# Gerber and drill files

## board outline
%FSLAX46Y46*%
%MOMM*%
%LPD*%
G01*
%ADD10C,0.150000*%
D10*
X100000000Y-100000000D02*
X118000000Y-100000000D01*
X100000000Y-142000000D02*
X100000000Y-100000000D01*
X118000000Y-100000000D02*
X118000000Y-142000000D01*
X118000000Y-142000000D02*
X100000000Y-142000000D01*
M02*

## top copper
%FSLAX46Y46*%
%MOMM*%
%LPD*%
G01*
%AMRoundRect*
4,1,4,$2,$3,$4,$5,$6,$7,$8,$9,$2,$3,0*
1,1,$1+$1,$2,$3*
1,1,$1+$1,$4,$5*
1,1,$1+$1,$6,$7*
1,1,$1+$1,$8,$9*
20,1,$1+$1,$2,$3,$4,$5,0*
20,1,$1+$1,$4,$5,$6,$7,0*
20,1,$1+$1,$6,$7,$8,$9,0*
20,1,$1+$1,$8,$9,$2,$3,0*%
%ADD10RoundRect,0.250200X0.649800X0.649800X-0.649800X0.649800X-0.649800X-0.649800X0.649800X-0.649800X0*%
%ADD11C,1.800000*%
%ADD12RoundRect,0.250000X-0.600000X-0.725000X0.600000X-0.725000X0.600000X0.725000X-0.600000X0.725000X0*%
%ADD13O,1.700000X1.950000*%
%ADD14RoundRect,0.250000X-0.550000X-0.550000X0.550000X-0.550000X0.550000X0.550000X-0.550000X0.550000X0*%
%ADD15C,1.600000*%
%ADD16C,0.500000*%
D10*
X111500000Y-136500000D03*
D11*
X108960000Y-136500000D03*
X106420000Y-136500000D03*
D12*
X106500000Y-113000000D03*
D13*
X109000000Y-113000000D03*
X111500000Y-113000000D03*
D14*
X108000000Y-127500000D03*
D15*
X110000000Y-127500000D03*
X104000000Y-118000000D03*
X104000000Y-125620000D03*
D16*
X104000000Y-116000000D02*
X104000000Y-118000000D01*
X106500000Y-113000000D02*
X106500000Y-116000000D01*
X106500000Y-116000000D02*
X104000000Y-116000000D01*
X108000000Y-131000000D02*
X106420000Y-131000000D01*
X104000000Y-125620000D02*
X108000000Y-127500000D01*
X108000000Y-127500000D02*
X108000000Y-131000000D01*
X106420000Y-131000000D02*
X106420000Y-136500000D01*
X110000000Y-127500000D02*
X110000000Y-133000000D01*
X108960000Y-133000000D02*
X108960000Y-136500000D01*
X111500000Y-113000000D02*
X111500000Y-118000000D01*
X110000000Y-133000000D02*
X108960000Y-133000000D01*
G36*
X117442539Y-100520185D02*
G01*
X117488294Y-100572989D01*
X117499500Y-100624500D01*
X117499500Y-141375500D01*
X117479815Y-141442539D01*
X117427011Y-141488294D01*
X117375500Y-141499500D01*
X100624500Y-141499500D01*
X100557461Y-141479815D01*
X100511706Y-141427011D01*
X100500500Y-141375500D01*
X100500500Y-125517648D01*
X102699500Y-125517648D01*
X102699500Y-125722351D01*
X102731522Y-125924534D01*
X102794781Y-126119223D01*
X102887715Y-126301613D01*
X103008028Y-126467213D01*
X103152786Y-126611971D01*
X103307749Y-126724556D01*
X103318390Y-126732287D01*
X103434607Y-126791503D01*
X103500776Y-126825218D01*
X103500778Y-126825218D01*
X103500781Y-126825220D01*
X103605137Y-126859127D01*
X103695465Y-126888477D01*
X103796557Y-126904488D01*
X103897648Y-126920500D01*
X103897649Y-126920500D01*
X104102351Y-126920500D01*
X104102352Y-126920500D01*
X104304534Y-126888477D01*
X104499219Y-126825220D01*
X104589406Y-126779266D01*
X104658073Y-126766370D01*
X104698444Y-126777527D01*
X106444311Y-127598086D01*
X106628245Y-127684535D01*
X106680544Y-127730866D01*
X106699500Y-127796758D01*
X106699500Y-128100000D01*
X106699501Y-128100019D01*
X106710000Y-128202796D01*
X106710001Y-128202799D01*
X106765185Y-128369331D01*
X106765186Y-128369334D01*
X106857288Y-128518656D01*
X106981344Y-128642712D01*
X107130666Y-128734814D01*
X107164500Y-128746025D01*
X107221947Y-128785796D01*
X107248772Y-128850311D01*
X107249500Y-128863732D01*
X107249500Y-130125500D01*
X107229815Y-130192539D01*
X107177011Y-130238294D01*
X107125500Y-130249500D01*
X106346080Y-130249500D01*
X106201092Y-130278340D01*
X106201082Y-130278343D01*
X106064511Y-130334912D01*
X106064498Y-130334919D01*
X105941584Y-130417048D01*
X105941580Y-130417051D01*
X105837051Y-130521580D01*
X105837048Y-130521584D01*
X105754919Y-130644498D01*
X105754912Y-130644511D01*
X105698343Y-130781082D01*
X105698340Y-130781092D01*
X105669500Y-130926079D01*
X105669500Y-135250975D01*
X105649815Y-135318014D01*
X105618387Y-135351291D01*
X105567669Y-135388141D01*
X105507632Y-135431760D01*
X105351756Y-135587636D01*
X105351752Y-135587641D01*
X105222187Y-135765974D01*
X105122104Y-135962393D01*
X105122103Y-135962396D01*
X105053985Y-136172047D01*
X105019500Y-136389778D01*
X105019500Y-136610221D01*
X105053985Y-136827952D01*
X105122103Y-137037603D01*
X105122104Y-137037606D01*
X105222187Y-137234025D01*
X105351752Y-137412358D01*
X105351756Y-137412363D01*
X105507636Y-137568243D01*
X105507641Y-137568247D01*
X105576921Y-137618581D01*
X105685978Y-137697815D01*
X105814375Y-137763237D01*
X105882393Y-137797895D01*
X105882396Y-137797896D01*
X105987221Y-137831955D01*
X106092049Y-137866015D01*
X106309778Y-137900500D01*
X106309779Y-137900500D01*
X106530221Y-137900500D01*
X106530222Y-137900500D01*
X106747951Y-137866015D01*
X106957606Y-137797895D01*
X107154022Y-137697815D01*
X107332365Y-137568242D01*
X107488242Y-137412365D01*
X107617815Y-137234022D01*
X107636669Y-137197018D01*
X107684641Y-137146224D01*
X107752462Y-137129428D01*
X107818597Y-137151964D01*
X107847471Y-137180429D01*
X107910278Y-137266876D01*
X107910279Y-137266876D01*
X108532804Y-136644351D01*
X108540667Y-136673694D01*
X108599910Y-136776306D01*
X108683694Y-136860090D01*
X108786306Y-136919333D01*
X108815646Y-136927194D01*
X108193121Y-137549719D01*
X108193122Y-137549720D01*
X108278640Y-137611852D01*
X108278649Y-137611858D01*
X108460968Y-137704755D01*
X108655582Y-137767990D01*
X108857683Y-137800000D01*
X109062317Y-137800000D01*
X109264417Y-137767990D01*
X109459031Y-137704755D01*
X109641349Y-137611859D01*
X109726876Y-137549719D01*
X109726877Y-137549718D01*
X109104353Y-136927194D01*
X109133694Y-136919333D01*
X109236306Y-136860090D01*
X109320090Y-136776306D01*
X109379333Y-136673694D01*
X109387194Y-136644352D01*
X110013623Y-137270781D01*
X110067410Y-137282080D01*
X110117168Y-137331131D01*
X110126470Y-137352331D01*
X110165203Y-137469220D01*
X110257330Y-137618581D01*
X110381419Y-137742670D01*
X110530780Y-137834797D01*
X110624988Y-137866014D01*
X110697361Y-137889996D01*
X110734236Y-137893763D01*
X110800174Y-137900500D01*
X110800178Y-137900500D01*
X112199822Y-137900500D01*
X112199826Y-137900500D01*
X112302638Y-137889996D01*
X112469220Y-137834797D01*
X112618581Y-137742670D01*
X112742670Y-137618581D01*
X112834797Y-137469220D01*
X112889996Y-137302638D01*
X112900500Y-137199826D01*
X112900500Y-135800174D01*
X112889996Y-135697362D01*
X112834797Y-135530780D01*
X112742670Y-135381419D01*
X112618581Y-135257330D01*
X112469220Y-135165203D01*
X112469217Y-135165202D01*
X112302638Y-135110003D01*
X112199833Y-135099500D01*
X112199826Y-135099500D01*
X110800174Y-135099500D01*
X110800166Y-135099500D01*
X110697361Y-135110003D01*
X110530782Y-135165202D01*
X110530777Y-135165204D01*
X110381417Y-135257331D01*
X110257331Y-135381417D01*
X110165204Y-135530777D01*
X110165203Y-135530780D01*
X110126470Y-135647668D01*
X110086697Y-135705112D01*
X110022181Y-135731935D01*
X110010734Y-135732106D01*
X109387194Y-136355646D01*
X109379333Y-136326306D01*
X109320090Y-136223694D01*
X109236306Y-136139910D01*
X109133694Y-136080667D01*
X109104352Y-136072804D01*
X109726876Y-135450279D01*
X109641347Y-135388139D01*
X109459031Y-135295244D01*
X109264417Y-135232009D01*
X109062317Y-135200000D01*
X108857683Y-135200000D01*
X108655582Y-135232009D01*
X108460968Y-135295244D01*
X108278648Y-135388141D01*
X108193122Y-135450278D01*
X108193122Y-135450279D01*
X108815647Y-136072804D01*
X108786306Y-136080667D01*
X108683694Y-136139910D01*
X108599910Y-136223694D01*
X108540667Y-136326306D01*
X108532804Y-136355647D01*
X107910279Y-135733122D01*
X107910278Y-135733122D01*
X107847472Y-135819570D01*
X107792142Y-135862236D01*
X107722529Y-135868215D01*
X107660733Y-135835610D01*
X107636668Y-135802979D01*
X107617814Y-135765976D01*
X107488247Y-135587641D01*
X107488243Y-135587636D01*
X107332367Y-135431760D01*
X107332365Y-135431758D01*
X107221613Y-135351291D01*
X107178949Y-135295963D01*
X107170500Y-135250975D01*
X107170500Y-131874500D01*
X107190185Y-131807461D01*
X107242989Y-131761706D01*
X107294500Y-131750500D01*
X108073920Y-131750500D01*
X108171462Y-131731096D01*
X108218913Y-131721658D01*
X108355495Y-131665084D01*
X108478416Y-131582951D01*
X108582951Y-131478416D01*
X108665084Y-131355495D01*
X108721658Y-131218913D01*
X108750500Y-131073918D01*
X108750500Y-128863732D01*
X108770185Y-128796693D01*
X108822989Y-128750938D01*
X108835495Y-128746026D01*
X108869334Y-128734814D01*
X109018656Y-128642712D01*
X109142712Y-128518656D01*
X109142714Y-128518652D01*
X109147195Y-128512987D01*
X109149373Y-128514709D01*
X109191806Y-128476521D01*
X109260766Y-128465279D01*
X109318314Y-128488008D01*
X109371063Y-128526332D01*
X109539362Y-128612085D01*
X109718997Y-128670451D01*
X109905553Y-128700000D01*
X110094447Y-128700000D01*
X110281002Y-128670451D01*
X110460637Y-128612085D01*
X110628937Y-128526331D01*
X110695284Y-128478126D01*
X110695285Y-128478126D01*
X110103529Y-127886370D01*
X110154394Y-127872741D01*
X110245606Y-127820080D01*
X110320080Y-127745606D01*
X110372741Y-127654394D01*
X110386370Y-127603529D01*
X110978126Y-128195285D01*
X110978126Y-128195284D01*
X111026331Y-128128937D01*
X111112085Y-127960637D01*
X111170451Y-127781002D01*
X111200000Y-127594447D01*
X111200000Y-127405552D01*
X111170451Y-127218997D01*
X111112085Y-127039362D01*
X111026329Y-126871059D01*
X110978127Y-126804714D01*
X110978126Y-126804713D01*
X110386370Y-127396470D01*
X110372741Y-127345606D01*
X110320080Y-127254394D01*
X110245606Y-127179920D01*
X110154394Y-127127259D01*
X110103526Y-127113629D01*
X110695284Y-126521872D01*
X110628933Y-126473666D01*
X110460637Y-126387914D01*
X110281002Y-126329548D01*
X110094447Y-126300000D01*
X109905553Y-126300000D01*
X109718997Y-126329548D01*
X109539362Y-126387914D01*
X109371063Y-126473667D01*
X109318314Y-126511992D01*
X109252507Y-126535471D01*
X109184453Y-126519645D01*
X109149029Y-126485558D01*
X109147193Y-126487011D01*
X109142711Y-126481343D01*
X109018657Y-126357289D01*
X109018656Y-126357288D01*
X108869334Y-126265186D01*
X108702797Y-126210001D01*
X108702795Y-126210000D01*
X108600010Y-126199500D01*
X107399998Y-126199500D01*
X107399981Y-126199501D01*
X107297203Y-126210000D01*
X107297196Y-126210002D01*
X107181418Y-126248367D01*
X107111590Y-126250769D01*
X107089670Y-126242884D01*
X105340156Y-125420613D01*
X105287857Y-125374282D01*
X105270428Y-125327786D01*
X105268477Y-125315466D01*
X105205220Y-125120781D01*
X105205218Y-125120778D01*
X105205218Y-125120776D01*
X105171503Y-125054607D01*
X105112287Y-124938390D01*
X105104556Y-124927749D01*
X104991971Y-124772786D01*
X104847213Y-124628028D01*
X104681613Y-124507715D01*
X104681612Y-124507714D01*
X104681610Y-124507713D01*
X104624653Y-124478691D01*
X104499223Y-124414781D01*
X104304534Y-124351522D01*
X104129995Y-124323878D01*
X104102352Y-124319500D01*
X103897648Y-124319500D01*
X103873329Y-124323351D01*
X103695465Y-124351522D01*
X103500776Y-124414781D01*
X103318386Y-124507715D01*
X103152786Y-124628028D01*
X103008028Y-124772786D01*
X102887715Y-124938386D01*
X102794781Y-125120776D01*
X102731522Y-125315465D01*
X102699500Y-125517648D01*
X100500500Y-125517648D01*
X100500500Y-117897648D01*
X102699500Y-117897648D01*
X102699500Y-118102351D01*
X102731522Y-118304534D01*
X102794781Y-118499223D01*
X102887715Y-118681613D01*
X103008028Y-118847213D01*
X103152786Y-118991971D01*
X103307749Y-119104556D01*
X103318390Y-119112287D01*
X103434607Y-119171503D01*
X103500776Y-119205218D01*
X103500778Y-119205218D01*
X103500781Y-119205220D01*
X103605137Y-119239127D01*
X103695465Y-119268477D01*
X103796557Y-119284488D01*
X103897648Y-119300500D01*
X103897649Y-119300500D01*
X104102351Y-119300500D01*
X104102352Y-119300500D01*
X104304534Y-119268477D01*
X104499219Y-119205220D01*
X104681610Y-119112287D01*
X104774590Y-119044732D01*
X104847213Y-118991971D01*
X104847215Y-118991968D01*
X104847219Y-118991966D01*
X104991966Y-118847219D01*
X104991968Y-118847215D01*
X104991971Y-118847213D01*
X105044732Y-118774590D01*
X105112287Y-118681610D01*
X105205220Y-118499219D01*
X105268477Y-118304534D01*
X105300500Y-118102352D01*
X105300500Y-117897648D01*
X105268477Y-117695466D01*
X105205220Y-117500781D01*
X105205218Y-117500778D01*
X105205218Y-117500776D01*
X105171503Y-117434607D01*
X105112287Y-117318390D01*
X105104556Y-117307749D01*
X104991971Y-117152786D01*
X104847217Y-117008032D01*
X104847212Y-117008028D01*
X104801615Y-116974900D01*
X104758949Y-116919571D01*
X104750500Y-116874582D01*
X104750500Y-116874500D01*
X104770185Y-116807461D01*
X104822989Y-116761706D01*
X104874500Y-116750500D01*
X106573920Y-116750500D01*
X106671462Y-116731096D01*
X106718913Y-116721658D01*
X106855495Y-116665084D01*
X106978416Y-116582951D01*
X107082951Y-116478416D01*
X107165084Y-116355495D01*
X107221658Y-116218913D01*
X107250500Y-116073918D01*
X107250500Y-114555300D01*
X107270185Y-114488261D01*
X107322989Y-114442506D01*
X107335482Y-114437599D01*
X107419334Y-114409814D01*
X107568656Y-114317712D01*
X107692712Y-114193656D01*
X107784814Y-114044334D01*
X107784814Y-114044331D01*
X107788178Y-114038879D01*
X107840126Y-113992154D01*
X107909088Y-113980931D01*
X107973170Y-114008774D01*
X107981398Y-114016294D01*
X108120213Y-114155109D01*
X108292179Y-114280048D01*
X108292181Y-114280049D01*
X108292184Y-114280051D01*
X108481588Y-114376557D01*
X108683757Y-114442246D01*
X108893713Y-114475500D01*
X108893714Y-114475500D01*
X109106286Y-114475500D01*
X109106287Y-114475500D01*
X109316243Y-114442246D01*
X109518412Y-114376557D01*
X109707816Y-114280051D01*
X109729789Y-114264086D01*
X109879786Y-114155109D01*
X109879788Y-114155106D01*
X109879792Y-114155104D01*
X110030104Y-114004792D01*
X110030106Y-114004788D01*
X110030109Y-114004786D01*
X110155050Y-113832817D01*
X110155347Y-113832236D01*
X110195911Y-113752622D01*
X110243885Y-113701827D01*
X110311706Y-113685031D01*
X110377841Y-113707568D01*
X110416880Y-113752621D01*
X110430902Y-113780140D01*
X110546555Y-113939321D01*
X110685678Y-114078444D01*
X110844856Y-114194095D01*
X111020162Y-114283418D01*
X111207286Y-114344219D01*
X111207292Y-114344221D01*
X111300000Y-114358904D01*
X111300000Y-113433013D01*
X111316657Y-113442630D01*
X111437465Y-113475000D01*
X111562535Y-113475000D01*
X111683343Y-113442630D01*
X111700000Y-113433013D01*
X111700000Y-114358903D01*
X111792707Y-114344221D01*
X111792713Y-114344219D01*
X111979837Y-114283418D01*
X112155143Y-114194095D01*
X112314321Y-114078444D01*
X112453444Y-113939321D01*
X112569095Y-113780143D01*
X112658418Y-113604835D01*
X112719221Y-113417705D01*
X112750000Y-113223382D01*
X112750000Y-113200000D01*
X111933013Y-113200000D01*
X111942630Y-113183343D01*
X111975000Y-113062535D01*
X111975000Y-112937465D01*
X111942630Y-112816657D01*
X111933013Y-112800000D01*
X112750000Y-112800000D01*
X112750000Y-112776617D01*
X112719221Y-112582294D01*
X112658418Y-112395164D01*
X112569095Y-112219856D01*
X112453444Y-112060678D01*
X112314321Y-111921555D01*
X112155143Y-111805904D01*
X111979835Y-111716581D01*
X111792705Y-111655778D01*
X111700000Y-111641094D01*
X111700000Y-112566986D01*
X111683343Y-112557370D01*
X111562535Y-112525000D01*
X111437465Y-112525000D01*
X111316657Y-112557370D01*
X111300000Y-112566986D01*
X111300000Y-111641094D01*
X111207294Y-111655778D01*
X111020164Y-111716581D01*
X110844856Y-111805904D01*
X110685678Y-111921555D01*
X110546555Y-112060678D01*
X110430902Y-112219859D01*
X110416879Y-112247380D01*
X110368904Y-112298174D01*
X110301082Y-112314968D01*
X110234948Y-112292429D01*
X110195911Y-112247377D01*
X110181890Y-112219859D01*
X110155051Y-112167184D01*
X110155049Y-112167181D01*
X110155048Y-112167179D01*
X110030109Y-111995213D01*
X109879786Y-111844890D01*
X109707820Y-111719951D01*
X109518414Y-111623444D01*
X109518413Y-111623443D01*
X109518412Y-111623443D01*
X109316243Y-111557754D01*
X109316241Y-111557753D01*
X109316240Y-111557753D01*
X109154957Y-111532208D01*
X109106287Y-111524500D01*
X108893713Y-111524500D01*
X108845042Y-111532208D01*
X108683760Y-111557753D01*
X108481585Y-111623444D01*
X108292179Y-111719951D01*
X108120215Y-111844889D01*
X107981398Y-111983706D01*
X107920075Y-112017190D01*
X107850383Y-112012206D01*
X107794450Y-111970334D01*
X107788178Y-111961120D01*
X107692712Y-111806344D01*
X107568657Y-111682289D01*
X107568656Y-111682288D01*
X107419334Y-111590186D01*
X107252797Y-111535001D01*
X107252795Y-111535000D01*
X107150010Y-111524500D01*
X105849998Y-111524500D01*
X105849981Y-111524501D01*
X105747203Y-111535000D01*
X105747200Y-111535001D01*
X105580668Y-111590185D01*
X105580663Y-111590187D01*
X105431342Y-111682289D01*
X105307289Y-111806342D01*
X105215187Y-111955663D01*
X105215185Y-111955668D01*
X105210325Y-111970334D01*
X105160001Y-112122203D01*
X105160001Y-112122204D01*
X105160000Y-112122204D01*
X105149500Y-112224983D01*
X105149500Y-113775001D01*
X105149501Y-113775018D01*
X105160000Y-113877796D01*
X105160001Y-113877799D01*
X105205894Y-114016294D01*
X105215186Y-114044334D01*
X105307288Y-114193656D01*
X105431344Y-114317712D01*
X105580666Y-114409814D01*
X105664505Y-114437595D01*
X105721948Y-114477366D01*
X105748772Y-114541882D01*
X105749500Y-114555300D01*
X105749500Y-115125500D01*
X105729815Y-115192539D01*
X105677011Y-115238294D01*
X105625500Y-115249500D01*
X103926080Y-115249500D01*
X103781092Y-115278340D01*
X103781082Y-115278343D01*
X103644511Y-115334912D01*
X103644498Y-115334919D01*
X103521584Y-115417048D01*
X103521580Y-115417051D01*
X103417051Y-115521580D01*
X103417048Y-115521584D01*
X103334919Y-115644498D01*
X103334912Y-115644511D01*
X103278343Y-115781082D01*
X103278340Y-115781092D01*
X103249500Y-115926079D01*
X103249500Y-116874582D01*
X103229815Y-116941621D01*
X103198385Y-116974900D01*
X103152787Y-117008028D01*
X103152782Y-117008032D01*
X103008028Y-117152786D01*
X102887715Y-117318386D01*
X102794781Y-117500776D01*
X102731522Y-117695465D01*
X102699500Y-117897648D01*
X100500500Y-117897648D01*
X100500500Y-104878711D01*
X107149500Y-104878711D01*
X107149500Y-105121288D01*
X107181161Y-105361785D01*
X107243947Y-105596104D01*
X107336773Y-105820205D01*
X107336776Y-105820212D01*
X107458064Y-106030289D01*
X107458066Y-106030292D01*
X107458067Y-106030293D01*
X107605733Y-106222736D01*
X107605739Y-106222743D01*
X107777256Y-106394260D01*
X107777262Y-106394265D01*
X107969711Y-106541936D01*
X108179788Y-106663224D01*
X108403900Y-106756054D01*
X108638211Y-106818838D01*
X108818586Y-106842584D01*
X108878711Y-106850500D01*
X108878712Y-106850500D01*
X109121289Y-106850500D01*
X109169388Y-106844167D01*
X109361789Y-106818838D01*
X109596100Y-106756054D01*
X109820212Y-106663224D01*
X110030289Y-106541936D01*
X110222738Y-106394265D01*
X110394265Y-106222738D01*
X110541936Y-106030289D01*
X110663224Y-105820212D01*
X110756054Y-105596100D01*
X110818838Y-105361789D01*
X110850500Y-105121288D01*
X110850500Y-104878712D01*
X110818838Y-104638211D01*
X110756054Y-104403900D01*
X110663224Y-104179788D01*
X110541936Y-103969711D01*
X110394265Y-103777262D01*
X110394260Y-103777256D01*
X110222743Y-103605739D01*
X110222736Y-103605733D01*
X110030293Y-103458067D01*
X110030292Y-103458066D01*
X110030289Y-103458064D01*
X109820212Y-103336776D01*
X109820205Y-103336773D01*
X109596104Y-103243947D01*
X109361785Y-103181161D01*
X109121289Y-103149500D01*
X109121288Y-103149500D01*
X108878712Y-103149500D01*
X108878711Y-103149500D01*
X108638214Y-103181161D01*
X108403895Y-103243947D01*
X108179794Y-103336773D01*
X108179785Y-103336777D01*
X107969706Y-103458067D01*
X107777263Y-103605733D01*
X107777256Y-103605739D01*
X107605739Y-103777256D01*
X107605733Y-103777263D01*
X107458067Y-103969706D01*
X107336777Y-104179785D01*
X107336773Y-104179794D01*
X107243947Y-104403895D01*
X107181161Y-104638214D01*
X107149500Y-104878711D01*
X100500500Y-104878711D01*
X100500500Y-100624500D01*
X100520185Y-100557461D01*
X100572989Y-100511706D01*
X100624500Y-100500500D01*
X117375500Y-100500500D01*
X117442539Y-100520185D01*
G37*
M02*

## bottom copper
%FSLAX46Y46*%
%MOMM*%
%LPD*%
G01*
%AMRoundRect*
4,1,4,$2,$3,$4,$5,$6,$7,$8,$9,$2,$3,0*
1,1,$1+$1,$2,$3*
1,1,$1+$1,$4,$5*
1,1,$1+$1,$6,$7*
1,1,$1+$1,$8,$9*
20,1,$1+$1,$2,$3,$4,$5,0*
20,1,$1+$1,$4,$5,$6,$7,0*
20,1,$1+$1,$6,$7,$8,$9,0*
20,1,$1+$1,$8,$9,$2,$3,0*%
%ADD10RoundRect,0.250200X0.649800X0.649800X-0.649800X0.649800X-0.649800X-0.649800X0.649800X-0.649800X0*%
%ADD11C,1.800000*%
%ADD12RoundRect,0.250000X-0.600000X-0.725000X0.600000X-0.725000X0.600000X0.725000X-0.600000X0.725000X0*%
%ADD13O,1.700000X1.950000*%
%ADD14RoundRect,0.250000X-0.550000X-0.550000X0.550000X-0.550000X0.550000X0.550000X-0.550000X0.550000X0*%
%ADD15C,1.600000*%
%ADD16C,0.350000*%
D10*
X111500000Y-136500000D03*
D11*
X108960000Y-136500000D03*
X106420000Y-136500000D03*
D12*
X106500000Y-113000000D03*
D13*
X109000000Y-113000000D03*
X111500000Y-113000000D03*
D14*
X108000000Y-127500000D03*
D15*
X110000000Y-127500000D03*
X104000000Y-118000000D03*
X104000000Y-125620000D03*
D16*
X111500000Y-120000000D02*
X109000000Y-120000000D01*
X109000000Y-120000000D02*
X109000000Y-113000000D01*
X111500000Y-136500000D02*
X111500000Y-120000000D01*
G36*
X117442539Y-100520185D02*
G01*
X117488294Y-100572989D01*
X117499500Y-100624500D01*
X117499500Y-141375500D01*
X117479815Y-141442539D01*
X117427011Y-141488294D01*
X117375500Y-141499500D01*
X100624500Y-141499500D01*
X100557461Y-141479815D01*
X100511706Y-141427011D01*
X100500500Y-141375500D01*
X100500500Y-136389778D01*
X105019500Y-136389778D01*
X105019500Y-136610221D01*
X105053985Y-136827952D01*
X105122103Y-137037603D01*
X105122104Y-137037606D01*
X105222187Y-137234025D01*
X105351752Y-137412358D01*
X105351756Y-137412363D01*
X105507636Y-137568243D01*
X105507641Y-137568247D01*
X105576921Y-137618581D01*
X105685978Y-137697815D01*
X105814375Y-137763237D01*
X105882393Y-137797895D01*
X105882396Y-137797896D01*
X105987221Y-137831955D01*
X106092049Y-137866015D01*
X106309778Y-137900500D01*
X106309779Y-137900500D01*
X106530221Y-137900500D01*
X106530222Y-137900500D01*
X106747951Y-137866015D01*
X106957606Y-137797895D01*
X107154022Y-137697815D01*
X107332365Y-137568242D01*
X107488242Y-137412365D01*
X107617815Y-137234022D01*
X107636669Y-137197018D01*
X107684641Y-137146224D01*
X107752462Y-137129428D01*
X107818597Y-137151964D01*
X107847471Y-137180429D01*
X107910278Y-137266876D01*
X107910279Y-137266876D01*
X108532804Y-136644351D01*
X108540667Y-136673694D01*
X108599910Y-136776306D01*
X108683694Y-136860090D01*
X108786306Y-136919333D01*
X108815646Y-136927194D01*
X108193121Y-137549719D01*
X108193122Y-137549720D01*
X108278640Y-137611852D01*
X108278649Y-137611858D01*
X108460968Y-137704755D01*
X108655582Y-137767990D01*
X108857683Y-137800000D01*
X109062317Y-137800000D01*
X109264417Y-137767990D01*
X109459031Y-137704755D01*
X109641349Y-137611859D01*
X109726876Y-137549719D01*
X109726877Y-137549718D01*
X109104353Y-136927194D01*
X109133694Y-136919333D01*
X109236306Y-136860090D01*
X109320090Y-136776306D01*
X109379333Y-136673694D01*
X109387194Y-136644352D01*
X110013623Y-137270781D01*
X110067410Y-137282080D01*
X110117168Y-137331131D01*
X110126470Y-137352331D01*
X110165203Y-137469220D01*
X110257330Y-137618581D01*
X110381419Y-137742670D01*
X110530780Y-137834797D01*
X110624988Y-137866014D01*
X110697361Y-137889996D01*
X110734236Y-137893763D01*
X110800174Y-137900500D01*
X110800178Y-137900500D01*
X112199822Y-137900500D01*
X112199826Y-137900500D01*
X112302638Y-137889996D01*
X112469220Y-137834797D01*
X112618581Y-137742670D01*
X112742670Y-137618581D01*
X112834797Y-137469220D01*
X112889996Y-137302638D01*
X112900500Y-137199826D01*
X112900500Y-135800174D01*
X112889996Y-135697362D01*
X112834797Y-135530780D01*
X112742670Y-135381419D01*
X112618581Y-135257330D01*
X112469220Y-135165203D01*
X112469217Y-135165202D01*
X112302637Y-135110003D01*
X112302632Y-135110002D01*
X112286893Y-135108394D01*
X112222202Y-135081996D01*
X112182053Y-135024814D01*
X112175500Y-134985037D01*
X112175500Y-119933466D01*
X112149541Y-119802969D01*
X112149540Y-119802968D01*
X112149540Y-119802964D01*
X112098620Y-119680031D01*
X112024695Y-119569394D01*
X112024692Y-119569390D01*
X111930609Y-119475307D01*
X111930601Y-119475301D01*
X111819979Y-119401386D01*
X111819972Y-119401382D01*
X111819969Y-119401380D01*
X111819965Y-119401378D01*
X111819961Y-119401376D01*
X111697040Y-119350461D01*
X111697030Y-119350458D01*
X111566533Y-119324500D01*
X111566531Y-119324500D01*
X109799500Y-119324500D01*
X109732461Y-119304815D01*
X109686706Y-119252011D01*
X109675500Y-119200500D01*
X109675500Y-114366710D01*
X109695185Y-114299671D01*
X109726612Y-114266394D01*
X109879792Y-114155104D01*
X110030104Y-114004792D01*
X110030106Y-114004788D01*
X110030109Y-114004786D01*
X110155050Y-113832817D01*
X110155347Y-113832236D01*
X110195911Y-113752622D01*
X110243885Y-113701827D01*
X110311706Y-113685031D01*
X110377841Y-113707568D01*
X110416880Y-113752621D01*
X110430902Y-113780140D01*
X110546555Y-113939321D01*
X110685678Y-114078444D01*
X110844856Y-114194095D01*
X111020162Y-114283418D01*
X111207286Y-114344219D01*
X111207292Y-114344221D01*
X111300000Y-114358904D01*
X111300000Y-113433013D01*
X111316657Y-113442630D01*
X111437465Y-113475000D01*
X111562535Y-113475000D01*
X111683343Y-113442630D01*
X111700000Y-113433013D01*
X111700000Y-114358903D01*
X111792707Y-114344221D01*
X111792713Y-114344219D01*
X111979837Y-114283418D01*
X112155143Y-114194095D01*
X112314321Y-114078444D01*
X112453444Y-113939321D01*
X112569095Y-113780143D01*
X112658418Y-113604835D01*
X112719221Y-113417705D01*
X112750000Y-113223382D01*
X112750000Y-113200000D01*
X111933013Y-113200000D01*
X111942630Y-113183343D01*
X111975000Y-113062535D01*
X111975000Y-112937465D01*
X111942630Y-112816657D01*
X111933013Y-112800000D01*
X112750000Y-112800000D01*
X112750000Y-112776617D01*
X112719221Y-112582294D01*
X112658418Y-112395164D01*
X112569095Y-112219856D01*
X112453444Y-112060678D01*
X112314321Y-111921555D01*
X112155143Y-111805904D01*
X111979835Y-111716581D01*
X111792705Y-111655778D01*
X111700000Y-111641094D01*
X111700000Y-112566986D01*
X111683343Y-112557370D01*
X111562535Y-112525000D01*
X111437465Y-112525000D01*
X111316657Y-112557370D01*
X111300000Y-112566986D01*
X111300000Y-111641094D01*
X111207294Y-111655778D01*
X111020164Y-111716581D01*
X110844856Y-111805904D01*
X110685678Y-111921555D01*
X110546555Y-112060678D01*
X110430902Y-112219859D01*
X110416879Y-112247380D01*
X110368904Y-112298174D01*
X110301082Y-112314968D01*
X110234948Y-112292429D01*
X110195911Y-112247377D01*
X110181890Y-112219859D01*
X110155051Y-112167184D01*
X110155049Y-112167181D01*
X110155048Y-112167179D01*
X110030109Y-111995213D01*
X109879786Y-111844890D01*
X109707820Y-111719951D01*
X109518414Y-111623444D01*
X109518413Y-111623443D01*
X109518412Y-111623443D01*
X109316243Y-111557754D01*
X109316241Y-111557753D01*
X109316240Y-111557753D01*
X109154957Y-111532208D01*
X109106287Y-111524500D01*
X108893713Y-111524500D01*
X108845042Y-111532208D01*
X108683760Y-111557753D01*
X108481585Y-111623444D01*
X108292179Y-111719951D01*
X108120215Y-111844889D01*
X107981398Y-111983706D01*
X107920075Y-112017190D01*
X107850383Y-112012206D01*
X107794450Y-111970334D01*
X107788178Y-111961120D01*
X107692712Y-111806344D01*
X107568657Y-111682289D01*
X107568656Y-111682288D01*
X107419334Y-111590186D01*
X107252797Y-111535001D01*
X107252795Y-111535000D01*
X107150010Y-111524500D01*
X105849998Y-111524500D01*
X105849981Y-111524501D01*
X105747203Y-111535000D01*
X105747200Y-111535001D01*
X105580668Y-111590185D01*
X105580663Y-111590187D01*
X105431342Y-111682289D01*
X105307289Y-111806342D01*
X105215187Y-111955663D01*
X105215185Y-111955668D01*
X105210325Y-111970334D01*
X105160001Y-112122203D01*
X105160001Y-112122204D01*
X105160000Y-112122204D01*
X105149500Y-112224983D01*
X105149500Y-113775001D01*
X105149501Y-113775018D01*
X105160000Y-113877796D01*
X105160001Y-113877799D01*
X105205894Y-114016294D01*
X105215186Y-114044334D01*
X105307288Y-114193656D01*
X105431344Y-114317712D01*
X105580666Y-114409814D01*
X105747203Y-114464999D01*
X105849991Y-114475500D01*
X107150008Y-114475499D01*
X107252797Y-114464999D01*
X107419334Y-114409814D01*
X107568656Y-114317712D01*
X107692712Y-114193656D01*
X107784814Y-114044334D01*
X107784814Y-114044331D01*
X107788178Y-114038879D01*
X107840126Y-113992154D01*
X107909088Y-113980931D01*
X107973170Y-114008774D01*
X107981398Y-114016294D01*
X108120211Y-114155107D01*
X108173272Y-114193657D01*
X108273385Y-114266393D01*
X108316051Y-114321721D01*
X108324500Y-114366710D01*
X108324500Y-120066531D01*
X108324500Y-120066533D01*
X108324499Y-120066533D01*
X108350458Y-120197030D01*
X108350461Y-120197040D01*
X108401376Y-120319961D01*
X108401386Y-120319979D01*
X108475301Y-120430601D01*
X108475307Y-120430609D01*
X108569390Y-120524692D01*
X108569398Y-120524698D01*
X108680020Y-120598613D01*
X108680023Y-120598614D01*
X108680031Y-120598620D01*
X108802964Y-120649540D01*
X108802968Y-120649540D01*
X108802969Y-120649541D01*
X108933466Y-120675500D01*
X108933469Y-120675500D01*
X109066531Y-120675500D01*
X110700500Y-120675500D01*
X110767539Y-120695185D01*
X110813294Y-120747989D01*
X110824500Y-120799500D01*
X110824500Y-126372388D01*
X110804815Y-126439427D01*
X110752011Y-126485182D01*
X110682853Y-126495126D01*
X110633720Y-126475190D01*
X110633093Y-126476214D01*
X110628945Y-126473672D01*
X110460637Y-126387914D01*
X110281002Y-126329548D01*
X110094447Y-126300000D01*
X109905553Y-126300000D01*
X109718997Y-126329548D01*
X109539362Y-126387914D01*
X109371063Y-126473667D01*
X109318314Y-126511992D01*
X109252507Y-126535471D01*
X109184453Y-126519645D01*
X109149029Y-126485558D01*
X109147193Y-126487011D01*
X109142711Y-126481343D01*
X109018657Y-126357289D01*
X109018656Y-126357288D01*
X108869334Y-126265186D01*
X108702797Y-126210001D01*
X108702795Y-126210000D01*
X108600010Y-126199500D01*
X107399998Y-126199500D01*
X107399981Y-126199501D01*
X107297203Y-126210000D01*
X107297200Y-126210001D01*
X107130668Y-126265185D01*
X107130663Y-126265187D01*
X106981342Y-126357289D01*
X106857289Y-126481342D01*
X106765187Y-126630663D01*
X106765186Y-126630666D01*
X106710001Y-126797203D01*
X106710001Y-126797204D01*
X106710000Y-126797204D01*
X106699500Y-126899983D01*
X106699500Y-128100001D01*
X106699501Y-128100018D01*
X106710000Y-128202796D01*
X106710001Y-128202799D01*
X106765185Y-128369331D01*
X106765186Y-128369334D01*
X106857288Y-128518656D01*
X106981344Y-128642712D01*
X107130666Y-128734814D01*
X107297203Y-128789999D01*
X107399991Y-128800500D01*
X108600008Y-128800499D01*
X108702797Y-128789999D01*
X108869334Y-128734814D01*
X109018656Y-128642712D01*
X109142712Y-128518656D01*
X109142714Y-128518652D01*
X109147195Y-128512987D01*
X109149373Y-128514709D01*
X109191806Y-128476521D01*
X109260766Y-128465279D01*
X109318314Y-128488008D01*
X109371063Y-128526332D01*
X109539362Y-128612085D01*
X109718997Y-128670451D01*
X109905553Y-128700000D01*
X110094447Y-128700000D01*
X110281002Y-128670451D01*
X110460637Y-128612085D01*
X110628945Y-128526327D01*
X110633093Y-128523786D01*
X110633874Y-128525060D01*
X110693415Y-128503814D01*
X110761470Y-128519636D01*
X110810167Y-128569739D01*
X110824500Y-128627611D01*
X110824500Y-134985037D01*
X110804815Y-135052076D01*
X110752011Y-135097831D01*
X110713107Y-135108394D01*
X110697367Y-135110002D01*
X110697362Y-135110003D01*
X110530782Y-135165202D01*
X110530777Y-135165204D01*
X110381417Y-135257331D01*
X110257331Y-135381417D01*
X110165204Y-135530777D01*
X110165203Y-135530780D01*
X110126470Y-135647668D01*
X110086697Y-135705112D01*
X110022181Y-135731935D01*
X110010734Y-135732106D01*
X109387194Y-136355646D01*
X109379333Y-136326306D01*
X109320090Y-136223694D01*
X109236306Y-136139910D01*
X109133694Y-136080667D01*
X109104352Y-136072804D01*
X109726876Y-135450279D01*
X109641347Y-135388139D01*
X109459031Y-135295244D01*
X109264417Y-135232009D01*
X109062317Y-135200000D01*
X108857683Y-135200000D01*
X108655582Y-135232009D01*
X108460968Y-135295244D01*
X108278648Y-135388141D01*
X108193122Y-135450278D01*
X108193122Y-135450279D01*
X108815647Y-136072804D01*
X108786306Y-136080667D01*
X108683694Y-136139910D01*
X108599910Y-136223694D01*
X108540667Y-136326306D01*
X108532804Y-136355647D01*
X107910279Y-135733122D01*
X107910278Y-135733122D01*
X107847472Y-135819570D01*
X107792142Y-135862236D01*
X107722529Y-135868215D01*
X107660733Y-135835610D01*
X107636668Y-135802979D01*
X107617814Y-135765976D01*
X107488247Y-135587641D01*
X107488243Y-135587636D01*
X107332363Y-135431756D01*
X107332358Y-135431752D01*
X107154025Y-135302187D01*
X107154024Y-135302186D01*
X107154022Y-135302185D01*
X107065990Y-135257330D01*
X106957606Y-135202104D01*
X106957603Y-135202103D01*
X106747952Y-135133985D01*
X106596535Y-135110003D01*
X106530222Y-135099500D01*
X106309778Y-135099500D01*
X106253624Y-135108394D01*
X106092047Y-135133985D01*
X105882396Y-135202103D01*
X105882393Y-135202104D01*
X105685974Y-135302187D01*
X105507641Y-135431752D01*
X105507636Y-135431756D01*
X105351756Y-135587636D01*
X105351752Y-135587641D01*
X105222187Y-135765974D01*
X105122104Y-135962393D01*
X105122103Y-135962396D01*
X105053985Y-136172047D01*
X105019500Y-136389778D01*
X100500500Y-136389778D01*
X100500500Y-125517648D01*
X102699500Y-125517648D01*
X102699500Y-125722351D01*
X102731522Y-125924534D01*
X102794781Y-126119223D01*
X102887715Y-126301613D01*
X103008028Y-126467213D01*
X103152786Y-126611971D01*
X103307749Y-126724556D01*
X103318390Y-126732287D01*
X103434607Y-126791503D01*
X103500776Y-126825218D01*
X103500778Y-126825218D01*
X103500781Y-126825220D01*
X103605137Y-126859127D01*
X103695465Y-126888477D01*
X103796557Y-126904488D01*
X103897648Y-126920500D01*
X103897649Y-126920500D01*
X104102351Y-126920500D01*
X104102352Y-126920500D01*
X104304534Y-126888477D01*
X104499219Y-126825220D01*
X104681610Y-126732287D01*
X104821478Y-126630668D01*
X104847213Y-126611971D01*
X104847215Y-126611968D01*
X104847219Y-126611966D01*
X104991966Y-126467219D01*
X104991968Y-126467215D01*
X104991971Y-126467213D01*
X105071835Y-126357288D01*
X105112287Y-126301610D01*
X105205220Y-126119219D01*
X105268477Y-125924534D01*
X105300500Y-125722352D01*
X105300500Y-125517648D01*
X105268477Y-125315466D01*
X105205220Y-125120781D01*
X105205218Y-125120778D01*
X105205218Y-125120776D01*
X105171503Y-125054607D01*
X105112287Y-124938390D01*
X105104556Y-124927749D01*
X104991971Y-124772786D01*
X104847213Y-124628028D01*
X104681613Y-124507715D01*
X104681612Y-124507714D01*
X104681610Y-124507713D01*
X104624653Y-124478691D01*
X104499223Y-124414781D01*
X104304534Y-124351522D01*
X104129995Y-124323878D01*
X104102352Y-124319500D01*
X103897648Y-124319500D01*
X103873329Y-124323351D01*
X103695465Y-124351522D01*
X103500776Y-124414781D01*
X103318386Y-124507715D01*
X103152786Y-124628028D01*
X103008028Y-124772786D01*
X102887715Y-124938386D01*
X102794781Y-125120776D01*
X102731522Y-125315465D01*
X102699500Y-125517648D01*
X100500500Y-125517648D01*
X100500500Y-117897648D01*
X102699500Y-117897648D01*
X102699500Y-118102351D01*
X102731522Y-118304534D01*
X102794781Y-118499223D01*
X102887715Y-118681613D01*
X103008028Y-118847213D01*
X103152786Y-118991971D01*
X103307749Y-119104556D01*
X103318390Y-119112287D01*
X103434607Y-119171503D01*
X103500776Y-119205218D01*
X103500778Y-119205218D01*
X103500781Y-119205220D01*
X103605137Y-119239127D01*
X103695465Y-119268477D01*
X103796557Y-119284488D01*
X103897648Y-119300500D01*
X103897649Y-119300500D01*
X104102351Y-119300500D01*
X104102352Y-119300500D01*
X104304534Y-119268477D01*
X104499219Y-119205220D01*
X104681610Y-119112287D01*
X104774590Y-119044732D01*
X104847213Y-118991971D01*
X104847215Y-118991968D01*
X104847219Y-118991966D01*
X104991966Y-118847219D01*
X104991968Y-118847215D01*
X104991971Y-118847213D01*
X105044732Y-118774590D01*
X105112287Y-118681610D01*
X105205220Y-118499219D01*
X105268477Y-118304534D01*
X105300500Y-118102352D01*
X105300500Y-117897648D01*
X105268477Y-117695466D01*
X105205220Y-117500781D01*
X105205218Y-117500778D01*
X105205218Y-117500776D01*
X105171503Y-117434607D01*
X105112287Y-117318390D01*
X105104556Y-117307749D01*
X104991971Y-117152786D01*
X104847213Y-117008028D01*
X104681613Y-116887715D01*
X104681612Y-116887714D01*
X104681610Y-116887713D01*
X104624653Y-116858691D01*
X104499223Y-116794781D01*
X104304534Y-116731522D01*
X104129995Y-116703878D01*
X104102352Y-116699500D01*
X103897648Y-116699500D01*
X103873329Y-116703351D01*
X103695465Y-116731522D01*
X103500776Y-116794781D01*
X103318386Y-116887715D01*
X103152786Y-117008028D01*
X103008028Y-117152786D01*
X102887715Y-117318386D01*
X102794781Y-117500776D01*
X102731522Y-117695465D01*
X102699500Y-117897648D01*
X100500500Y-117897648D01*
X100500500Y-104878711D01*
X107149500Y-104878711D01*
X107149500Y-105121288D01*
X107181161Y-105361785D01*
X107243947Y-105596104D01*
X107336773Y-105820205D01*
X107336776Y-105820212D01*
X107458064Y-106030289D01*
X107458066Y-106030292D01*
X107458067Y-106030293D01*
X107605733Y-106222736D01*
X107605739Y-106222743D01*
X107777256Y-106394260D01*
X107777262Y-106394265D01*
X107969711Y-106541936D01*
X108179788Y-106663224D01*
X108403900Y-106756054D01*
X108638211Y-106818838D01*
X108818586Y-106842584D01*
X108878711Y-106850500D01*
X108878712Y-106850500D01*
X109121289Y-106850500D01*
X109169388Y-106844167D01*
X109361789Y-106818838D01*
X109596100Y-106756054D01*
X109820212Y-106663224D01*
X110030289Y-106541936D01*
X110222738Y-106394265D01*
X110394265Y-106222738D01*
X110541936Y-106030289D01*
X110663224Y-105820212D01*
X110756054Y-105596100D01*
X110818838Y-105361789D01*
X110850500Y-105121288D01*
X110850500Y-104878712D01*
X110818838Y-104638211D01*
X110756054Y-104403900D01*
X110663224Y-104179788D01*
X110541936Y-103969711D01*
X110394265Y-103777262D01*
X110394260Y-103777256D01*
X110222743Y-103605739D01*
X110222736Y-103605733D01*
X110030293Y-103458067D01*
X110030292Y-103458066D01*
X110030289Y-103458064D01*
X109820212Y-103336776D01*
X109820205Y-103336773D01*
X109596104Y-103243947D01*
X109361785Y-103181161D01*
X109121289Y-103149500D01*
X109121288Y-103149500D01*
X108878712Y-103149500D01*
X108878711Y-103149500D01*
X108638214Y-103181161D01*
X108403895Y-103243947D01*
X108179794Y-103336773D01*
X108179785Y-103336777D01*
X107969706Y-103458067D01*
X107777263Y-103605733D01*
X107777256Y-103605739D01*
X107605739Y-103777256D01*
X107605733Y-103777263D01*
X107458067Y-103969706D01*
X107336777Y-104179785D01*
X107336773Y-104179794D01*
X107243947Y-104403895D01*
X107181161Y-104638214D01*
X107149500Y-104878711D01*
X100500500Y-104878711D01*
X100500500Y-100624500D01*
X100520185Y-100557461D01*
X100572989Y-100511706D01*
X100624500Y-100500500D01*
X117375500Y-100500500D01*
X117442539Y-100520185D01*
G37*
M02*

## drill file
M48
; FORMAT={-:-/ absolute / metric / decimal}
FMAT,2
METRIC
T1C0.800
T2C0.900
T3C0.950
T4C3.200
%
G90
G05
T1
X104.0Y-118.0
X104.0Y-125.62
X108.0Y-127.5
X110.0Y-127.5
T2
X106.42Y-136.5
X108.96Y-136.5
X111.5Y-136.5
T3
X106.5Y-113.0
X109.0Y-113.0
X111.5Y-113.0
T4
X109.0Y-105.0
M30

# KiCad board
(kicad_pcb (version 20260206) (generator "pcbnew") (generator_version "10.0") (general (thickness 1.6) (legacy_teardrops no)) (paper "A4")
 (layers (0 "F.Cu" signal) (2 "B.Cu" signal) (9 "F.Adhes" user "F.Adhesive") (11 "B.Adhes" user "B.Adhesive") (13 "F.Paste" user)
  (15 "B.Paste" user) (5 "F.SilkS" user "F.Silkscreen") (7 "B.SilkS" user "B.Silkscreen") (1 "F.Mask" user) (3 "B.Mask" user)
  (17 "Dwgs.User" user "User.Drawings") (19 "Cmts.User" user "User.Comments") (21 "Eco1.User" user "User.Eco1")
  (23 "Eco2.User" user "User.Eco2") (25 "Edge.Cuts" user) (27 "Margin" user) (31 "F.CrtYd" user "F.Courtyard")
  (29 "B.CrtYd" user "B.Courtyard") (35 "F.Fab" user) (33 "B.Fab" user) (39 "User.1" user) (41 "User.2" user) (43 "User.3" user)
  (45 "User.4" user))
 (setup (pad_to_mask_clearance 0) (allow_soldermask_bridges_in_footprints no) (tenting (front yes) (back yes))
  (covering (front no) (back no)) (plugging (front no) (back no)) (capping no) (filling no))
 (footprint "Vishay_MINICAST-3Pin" (layer "F.Cu") (at 111.5 136.5 180)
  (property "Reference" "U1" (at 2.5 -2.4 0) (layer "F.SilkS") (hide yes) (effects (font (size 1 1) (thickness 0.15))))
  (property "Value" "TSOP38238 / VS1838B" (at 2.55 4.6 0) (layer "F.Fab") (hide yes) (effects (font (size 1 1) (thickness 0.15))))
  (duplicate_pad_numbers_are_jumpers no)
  (pad "1" thru_hole roundrect (at 0 0 180) (size 1.8 1.8) (drill 0.9) (layers "*.Cu" "*.Mask") (remove_unused_layers no)
   (roundrect_rratio 0.139) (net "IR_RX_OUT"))
  (pad "2" thru_hole circle (at 2.54 0 180) (size 1.8 1.8) (drill 0.9) (layers "*.Cu" "*.Mask") (remove_unused_layers no) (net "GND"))
  (pad "3" thru_hole circle (at 5.08 0 180) (size 1.8 1.8) (drill 0.9) (layers "*.Cu" "*.Mask") (remove_unused_layers no) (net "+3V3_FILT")))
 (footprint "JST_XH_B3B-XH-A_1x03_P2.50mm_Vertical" (layer "F.Cu") (at 106.5 113)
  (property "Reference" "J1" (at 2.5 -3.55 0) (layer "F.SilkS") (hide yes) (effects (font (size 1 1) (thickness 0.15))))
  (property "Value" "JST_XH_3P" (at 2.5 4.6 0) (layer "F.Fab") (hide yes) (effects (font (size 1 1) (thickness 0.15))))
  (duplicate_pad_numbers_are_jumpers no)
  (pad "1" thru_hole roundrect (at 0 0) (size 1.7 1.95) (drill 0.95) (layers "*.Cu" "*.Mask") (remove_unused_layers no)
   (roundrect_rratio 0.147059) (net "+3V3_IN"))
  (pad "2" thru_hole oval (at 2.5 0) (size 1.7 1.95) (drill 0.95) (layers "*.Cu" "*.Mask") (remove_unused_layers no) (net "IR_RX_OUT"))
  (pad "3" thru_hole oval (at 5 0) (size 1.7 1.95) (drill 0.95) (layers "*.Cu" "*.Mask") (remove_unused_layers no) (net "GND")))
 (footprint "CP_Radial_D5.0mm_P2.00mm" (layer "F.Cu") (at 108 127.5)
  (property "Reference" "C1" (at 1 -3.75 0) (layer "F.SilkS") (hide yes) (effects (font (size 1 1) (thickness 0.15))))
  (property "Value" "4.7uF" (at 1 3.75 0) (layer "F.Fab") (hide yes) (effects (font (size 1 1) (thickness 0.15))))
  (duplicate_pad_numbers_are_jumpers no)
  (pad "1" thru_hole roundrect (at 0 0) (size 1.6 1.6) (drill 0.8) (layers "*.Cu" "*.Mask") (remove_unused_layers no)
   (roundrect_rratio 0.15625) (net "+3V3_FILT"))
  (pad "2" thru_hole circle (at 2 0) (size 1.6 1.6) (drill 0.8) (layers "*.Cu" "*.Mask") (remove_unused_layers no) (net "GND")))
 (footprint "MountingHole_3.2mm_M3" (layer "F.Cu") (at 109 105)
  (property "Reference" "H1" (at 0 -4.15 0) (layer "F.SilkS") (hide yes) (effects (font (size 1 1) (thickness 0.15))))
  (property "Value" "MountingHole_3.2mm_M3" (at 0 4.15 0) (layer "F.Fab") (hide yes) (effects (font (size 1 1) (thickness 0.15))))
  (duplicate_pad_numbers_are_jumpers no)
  (pad "" np_thru_hole circle (at 0 0) (size 3.2 3.2) (drill 3.2) (layers "*.Cu" "*.Mask")))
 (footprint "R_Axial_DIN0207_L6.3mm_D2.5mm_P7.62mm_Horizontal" (layer "F.Cu") (at 104 118 -90)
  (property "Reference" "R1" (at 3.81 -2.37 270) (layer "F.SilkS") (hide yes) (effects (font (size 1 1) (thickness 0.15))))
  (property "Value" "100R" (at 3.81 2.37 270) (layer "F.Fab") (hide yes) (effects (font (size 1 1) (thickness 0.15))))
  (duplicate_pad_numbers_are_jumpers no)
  (pad "1" thru_hole circle (at 0 0 270) (size 1.6 1.6) (drill 0.8) (layers "*.Cu" "*.Mask") (remove_unused_layers no) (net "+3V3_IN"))
  (pad "2" thru_hole circle (at 7.62 0 270) (size 1.6 1.6) (drill 0.8) (layers "*.Cu" "*.Mask") (remove_unused_layers no) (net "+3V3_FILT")))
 (gr_line (start 100 100) (end 118 100) (stroke (width 0.15) (type default)) (layer "Edge.Cuts"))
 (gr_line (start 100 142) (end 100 100) (stroke (width 0.15) (type default)) (layer "Edge.Cuts"))
 (gr_line (start 118 100) (end 118 142) (stroke (width 0.15) (type default)) (layer "Edge.Cuts"))
 (gr_line (start 118 142) (end 100 142) (stroke (width 0.15) (type default)) (layer "Edge.Cuts"))
 (segment (start 104 116) (end 104 118) (width 0.5) (layer "F.Cu") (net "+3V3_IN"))
 (segment (start 106.5 113) (end 106.5 116) (width 0.5) (layer "F.Cu") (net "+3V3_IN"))
 (segment (start 106.5 116) (end 104 116) (width 0.5) (layer "F.Cu") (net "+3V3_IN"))
 (segment (start 108 131) (end 106.42 131) (width 0.5) (layer "F.Cu") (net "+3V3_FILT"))
 (segment (start 104 125.62) (end 108 127.5) (width 0.5) (layer "F.Cu") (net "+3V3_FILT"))
 (segment (start 108 127.5) (end 108 131) (width 0.5) (layer "F.Cu") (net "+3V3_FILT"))
 (segment (start 106.42 131) (end 106.42 136.5) (width 0.5) (layer "F.Cu") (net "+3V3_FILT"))
 (segment (start 111.5 120) (end 109 120) (width 0.35) (layer "B.Cu") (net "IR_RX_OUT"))
 (segment (start 109 120) (end 109 113) (width 0.35) (layer "B.Cu") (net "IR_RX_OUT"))
 (segment (start 111.5 136.5) (end 111.5 120) (width 0.35) (layer "B.Cu") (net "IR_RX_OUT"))
 (segment (start 110 127.5) (end 110 133) (width 0.5) (layer "F.Cu") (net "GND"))
 (segment (start 108.96 133) (end 108.96 136.5) (width 0.5) (layer "F.Cu") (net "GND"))
 (segment (start 111.5 113) (end 111.5 118) (width 0.5) (layer "F.Cu") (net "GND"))
 (segment (start 110 133) (end 108.96 133) (width 0.5) (layer "F.Cu") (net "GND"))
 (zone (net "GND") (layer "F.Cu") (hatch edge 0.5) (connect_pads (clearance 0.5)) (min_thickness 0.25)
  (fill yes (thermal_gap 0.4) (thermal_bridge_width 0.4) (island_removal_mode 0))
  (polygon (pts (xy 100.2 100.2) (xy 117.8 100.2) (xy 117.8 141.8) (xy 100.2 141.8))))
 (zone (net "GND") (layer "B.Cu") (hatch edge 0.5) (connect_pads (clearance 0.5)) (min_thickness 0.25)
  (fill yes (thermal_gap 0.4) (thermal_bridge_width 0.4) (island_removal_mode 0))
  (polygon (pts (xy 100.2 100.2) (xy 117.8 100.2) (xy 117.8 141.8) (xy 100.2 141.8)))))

